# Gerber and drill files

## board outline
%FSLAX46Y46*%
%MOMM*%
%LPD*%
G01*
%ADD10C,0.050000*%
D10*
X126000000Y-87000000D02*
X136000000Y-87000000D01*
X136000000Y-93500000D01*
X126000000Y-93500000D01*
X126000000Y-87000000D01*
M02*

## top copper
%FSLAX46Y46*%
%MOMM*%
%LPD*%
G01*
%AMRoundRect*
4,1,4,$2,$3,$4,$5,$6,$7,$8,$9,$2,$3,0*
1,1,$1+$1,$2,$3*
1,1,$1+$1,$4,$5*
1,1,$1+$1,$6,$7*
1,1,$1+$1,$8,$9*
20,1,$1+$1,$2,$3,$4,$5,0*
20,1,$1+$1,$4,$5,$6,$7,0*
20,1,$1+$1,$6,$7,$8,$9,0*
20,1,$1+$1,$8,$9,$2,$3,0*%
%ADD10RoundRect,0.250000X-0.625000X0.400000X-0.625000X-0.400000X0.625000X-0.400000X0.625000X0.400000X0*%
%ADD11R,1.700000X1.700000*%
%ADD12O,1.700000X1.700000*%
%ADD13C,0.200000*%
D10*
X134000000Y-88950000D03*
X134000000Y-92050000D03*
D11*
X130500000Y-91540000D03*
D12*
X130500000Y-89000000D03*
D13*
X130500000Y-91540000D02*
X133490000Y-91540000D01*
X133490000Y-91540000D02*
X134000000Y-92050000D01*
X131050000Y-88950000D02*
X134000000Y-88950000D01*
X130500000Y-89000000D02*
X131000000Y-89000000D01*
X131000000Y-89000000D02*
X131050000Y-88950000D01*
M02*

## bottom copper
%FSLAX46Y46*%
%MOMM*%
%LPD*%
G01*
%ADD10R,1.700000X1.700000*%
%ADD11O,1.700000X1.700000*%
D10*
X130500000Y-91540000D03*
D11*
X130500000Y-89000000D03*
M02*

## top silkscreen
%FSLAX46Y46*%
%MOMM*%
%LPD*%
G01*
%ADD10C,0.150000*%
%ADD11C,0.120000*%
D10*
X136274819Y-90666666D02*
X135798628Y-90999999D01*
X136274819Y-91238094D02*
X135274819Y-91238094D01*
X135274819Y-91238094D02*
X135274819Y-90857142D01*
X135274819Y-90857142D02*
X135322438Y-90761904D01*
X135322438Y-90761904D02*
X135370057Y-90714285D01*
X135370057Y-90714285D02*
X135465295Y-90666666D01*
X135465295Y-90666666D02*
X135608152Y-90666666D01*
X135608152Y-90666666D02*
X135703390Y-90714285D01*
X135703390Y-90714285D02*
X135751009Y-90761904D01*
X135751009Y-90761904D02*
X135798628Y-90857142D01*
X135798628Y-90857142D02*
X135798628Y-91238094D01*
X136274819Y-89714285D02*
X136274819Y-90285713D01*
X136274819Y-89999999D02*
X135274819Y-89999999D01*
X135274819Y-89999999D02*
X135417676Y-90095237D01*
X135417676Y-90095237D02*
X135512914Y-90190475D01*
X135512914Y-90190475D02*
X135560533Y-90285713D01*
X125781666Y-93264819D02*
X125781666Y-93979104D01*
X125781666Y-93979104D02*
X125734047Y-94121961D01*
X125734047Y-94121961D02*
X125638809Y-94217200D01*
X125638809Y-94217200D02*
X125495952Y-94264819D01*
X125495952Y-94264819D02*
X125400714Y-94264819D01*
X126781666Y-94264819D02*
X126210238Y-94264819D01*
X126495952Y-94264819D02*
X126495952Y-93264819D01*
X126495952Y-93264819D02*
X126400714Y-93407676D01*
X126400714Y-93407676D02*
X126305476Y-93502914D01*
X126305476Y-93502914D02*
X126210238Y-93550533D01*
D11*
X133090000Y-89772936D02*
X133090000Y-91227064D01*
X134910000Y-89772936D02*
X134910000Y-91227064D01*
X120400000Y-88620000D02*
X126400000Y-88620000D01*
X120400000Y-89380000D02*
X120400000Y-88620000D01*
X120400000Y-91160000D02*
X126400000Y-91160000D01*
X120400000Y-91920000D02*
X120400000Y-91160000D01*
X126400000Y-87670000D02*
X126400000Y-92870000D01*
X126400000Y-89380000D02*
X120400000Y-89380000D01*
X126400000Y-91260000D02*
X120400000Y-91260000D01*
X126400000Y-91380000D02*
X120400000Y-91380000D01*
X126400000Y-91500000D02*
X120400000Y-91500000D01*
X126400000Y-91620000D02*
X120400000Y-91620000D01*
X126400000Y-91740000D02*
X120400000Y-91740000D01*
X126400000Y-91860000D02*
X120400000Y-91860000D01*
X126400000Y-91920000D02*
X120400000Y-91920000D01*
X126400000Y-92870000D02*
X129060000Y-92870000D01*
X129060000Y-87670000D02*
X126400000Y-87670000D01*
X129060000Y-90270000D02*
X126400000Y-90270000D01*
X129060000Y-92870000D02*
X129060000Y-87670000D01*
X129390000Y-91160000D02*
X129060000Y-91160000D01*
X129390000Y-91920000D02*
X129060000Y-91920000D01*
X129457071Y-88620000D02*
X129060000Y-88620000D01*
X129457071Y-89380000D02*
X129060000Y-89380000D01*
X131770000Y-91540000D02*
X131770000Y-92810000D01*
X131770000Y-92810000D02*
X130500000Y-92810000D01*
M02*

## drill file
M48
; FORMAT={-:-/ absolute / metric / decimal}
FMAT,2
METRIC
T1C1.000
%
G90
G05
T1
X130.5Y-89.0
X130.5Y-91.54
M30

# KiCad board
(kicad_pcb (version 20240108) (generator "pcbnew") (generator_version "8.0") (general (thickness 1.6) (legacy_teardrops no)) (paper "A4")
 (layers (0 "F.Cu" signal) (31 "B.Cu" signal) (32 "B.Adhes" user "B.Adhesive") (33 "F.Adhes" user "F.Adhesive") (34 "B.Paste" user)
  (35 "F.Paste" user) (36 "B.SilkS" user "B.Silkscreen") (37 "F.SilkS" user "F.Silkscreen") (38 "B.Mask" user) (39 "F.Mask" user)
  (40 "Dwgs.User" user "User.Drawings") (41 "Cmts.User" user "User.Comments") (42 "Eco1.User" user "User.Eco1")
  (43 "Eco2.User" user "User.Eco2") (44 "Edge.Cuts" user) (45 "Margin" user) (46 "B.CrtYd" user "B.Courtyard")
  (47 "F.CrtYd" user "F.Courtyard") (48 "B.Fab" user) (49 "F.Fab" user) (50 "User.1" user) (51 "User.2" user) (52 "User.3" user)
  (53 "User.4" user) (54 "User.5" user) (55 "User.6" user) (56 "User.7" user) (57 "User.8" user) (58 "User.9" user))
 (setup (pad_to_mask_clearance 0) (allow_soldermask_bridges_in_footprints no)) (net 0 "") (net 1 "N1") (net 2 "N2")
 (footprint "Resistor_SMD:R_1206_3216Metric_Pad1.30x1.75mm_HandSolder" (layer "F.Cu") (at 134 90.5 -90)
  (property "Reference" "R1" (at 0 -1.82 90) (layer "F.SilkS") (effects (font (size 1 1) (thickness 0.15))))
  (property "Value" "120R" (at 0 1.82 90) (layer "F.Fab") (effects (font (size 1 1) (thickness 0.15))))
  (fp_line (start -0.727064 0.91) (end 0.727064 0.91) (stroke (width 0.12) (type solid)) (layer "F.SilkS"))
  (fp_line (start -0.727064 -0.91) (end 0.727064 -0.91) (stroke (width 0.12) (type solid)) (layer "F.SilkS"))
  (pad "1" smd roundrect (at -1.55 0 270) (size 1.3 1.75) (layers "F.Cu" "F.Paste" "F.Mask") (roundrect_rratio 0.192308) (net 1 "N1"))
  (pad "2" smd roundrect (at 1.55 0 270) (size 1.3 1.75) (layers "F.Cu" "F.Paste" "F.Mask") (roundrect_rratio 0.192308) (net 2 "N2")))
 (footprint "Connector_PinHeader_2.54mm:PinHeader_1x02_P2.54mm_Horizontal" (layer "F.Cu") (at 130.5 91.54 180)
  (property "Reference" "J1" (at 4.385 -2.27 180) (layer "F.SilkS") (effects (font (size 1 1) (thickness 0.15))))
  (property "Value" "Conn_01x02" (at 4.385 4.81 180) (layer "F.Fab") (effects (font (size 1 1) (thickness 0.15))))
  (fp_line (start 10.1 2.92) (end 4.1 2.92) (stroke (width 0.12) (type solid)) (layer "F.SilkS"))
  (fp_line (start 10.1 2.16) (end 10.1 2.92) (stroke (width 0.12) (type solid)) (layer "F.SilkS"))
  (fp_line (start 10.1 0.38) (end 4.1 0.38) (stroke (width 0.12) (type solid)) (layer "F.SilkS"))
  (fp_line (start 10.1 -0.38) (end 10.1 0.38) (stroke (width 0.12) (type solid)) (layer "F.SilkS"))
  (fp_line (start 4.1 3.87) (end 4.1 -1.33) (stroke (width 0.12) (type solid)) (layer "F.SilkS"))
  (fp_line (start 4.1 2.16) (end 10.1 2.16) (stroke (width 0.12) (type solid)) (layer "F.SilkS"))
  (fp_line (start 4.1 0.28) (end 10.1 0.28) (stroke (width 0.12) (type solid)) (layer "F.SilkS"))
  (fp_line (start 4.1 0.16) (end 10.1 0.16) (stroke (width 0.12) (type solid)) (layer "F.SilkS"))
  (fp_line (start 4.1 0.04) (end 10.1 0.04) (stroke (width 0.12) (type solid)) (layer "F.SilkS"))
  (fp_line (start 4.1 -0.08) (end 10.1 -0.08) (stroke (width 0.12) (type solid)) (layer "F.SilkS"))
  (fp_line (start 4.1 -0.2) (end 10.1 -0.2) (stroke (width 0.12) (type solid)) (layer "F.SilkS"))
  (fp_line (start 4.1 -0.32) (end 10.1 -0.32) (stroke (width 0.12) (type solid)) (layer "F.SilkS"))
  (fp_line (start 4.1 -0.38) (end 10.1 -0.38) (stroke (width 0.12) (type solid)) (layer "F.SilkS"))
  (fp_line (start 4.1 -1.33) (end 1.44 -1.33) (stroke (width 0.12) (type solid)) (layer "F.SilkS"))
  (fp_line (start 1.44 3.87) (end 4.1 3.87) (stroke (width 0.12) (type solid)) (layer "F.SilkS"))
  (fp_line (start 1.44 1.27) (end 4.1 1.27) (stroke (width 0.12) (type solid)) (layer "F.SilkS"))
  (fp_line (start 1.44 -1.33) (end 1.44 3.87) (stroke (width 0.12) (type solid)) (layer "F.SilkS"))
  (fp_line (start 1.11 0.38) (end 1.44 0.38) (stroke (width 0.12) (type solid)) (layer "F.SilkS"))
  (fp_line (start 1.11 -0.38) (end 1.44 -0.38) (stroke (width 0.12) (type solid)) (layer "F.SilkS"))
  (fp_line (start 1.042929 2.92) (end 1.44 2.92) (stroke (width 0.12) (type solid)) (layer "F.SilkS"))
  (fp_line (start 1.042929 2.16) (end 1.44 2.16) (stroke (width 0.12) (type solid)) (layer "F.SilkS"))
  (fp_line (start -1.27 0) (end -1.27 -1.27) (stroke (width 0.12) (type solid)) (layer "F.SilkS"))
  (fp_line (start -1.27 -1.27) (end 0 -1.27) (stroke (width 0.12) (type solid)) (layer "F.SilkS"))
  (pad "1" thru_hole rect (at 0 0 180) (size 1.7 1.7) (drill 1) (layers "*.Cu" "*.Mask") (remove_unused_layers no) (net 2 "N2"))
  (pad "2" thru_hole oval (at 0 2.54 180) (size 1.7 1.7) (drill 1) (layers "*.Cu" "*.Mask") (remove_unused_layers no) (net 1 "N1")))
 (gr_rect (start 126 87) (end 136 93.5) (stroke (width 0.05) (type default)) (fill none) (layer "Edge.Cuts"))
 (segment (start 130.5 91.54) (end 133.49 91.54) (width 0.2) (layer "F.Cu") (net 2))
 (segment (start 133.49 91.54) (end 134 92.05) (width 0.2) (layer "F.Cu") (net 2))
 (segment (start 131.05 88.95) (end 134 88.95) (width 0.2) (layer "F.Cu") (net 1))
 (segment (start 130.5 89) (end 131 89) (width 0.2) (layer "F.Cu") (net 1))
 (segment (start 131 89) (end 131.05 88.95) (width 0.2) (layer "F.Cu") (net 1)))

